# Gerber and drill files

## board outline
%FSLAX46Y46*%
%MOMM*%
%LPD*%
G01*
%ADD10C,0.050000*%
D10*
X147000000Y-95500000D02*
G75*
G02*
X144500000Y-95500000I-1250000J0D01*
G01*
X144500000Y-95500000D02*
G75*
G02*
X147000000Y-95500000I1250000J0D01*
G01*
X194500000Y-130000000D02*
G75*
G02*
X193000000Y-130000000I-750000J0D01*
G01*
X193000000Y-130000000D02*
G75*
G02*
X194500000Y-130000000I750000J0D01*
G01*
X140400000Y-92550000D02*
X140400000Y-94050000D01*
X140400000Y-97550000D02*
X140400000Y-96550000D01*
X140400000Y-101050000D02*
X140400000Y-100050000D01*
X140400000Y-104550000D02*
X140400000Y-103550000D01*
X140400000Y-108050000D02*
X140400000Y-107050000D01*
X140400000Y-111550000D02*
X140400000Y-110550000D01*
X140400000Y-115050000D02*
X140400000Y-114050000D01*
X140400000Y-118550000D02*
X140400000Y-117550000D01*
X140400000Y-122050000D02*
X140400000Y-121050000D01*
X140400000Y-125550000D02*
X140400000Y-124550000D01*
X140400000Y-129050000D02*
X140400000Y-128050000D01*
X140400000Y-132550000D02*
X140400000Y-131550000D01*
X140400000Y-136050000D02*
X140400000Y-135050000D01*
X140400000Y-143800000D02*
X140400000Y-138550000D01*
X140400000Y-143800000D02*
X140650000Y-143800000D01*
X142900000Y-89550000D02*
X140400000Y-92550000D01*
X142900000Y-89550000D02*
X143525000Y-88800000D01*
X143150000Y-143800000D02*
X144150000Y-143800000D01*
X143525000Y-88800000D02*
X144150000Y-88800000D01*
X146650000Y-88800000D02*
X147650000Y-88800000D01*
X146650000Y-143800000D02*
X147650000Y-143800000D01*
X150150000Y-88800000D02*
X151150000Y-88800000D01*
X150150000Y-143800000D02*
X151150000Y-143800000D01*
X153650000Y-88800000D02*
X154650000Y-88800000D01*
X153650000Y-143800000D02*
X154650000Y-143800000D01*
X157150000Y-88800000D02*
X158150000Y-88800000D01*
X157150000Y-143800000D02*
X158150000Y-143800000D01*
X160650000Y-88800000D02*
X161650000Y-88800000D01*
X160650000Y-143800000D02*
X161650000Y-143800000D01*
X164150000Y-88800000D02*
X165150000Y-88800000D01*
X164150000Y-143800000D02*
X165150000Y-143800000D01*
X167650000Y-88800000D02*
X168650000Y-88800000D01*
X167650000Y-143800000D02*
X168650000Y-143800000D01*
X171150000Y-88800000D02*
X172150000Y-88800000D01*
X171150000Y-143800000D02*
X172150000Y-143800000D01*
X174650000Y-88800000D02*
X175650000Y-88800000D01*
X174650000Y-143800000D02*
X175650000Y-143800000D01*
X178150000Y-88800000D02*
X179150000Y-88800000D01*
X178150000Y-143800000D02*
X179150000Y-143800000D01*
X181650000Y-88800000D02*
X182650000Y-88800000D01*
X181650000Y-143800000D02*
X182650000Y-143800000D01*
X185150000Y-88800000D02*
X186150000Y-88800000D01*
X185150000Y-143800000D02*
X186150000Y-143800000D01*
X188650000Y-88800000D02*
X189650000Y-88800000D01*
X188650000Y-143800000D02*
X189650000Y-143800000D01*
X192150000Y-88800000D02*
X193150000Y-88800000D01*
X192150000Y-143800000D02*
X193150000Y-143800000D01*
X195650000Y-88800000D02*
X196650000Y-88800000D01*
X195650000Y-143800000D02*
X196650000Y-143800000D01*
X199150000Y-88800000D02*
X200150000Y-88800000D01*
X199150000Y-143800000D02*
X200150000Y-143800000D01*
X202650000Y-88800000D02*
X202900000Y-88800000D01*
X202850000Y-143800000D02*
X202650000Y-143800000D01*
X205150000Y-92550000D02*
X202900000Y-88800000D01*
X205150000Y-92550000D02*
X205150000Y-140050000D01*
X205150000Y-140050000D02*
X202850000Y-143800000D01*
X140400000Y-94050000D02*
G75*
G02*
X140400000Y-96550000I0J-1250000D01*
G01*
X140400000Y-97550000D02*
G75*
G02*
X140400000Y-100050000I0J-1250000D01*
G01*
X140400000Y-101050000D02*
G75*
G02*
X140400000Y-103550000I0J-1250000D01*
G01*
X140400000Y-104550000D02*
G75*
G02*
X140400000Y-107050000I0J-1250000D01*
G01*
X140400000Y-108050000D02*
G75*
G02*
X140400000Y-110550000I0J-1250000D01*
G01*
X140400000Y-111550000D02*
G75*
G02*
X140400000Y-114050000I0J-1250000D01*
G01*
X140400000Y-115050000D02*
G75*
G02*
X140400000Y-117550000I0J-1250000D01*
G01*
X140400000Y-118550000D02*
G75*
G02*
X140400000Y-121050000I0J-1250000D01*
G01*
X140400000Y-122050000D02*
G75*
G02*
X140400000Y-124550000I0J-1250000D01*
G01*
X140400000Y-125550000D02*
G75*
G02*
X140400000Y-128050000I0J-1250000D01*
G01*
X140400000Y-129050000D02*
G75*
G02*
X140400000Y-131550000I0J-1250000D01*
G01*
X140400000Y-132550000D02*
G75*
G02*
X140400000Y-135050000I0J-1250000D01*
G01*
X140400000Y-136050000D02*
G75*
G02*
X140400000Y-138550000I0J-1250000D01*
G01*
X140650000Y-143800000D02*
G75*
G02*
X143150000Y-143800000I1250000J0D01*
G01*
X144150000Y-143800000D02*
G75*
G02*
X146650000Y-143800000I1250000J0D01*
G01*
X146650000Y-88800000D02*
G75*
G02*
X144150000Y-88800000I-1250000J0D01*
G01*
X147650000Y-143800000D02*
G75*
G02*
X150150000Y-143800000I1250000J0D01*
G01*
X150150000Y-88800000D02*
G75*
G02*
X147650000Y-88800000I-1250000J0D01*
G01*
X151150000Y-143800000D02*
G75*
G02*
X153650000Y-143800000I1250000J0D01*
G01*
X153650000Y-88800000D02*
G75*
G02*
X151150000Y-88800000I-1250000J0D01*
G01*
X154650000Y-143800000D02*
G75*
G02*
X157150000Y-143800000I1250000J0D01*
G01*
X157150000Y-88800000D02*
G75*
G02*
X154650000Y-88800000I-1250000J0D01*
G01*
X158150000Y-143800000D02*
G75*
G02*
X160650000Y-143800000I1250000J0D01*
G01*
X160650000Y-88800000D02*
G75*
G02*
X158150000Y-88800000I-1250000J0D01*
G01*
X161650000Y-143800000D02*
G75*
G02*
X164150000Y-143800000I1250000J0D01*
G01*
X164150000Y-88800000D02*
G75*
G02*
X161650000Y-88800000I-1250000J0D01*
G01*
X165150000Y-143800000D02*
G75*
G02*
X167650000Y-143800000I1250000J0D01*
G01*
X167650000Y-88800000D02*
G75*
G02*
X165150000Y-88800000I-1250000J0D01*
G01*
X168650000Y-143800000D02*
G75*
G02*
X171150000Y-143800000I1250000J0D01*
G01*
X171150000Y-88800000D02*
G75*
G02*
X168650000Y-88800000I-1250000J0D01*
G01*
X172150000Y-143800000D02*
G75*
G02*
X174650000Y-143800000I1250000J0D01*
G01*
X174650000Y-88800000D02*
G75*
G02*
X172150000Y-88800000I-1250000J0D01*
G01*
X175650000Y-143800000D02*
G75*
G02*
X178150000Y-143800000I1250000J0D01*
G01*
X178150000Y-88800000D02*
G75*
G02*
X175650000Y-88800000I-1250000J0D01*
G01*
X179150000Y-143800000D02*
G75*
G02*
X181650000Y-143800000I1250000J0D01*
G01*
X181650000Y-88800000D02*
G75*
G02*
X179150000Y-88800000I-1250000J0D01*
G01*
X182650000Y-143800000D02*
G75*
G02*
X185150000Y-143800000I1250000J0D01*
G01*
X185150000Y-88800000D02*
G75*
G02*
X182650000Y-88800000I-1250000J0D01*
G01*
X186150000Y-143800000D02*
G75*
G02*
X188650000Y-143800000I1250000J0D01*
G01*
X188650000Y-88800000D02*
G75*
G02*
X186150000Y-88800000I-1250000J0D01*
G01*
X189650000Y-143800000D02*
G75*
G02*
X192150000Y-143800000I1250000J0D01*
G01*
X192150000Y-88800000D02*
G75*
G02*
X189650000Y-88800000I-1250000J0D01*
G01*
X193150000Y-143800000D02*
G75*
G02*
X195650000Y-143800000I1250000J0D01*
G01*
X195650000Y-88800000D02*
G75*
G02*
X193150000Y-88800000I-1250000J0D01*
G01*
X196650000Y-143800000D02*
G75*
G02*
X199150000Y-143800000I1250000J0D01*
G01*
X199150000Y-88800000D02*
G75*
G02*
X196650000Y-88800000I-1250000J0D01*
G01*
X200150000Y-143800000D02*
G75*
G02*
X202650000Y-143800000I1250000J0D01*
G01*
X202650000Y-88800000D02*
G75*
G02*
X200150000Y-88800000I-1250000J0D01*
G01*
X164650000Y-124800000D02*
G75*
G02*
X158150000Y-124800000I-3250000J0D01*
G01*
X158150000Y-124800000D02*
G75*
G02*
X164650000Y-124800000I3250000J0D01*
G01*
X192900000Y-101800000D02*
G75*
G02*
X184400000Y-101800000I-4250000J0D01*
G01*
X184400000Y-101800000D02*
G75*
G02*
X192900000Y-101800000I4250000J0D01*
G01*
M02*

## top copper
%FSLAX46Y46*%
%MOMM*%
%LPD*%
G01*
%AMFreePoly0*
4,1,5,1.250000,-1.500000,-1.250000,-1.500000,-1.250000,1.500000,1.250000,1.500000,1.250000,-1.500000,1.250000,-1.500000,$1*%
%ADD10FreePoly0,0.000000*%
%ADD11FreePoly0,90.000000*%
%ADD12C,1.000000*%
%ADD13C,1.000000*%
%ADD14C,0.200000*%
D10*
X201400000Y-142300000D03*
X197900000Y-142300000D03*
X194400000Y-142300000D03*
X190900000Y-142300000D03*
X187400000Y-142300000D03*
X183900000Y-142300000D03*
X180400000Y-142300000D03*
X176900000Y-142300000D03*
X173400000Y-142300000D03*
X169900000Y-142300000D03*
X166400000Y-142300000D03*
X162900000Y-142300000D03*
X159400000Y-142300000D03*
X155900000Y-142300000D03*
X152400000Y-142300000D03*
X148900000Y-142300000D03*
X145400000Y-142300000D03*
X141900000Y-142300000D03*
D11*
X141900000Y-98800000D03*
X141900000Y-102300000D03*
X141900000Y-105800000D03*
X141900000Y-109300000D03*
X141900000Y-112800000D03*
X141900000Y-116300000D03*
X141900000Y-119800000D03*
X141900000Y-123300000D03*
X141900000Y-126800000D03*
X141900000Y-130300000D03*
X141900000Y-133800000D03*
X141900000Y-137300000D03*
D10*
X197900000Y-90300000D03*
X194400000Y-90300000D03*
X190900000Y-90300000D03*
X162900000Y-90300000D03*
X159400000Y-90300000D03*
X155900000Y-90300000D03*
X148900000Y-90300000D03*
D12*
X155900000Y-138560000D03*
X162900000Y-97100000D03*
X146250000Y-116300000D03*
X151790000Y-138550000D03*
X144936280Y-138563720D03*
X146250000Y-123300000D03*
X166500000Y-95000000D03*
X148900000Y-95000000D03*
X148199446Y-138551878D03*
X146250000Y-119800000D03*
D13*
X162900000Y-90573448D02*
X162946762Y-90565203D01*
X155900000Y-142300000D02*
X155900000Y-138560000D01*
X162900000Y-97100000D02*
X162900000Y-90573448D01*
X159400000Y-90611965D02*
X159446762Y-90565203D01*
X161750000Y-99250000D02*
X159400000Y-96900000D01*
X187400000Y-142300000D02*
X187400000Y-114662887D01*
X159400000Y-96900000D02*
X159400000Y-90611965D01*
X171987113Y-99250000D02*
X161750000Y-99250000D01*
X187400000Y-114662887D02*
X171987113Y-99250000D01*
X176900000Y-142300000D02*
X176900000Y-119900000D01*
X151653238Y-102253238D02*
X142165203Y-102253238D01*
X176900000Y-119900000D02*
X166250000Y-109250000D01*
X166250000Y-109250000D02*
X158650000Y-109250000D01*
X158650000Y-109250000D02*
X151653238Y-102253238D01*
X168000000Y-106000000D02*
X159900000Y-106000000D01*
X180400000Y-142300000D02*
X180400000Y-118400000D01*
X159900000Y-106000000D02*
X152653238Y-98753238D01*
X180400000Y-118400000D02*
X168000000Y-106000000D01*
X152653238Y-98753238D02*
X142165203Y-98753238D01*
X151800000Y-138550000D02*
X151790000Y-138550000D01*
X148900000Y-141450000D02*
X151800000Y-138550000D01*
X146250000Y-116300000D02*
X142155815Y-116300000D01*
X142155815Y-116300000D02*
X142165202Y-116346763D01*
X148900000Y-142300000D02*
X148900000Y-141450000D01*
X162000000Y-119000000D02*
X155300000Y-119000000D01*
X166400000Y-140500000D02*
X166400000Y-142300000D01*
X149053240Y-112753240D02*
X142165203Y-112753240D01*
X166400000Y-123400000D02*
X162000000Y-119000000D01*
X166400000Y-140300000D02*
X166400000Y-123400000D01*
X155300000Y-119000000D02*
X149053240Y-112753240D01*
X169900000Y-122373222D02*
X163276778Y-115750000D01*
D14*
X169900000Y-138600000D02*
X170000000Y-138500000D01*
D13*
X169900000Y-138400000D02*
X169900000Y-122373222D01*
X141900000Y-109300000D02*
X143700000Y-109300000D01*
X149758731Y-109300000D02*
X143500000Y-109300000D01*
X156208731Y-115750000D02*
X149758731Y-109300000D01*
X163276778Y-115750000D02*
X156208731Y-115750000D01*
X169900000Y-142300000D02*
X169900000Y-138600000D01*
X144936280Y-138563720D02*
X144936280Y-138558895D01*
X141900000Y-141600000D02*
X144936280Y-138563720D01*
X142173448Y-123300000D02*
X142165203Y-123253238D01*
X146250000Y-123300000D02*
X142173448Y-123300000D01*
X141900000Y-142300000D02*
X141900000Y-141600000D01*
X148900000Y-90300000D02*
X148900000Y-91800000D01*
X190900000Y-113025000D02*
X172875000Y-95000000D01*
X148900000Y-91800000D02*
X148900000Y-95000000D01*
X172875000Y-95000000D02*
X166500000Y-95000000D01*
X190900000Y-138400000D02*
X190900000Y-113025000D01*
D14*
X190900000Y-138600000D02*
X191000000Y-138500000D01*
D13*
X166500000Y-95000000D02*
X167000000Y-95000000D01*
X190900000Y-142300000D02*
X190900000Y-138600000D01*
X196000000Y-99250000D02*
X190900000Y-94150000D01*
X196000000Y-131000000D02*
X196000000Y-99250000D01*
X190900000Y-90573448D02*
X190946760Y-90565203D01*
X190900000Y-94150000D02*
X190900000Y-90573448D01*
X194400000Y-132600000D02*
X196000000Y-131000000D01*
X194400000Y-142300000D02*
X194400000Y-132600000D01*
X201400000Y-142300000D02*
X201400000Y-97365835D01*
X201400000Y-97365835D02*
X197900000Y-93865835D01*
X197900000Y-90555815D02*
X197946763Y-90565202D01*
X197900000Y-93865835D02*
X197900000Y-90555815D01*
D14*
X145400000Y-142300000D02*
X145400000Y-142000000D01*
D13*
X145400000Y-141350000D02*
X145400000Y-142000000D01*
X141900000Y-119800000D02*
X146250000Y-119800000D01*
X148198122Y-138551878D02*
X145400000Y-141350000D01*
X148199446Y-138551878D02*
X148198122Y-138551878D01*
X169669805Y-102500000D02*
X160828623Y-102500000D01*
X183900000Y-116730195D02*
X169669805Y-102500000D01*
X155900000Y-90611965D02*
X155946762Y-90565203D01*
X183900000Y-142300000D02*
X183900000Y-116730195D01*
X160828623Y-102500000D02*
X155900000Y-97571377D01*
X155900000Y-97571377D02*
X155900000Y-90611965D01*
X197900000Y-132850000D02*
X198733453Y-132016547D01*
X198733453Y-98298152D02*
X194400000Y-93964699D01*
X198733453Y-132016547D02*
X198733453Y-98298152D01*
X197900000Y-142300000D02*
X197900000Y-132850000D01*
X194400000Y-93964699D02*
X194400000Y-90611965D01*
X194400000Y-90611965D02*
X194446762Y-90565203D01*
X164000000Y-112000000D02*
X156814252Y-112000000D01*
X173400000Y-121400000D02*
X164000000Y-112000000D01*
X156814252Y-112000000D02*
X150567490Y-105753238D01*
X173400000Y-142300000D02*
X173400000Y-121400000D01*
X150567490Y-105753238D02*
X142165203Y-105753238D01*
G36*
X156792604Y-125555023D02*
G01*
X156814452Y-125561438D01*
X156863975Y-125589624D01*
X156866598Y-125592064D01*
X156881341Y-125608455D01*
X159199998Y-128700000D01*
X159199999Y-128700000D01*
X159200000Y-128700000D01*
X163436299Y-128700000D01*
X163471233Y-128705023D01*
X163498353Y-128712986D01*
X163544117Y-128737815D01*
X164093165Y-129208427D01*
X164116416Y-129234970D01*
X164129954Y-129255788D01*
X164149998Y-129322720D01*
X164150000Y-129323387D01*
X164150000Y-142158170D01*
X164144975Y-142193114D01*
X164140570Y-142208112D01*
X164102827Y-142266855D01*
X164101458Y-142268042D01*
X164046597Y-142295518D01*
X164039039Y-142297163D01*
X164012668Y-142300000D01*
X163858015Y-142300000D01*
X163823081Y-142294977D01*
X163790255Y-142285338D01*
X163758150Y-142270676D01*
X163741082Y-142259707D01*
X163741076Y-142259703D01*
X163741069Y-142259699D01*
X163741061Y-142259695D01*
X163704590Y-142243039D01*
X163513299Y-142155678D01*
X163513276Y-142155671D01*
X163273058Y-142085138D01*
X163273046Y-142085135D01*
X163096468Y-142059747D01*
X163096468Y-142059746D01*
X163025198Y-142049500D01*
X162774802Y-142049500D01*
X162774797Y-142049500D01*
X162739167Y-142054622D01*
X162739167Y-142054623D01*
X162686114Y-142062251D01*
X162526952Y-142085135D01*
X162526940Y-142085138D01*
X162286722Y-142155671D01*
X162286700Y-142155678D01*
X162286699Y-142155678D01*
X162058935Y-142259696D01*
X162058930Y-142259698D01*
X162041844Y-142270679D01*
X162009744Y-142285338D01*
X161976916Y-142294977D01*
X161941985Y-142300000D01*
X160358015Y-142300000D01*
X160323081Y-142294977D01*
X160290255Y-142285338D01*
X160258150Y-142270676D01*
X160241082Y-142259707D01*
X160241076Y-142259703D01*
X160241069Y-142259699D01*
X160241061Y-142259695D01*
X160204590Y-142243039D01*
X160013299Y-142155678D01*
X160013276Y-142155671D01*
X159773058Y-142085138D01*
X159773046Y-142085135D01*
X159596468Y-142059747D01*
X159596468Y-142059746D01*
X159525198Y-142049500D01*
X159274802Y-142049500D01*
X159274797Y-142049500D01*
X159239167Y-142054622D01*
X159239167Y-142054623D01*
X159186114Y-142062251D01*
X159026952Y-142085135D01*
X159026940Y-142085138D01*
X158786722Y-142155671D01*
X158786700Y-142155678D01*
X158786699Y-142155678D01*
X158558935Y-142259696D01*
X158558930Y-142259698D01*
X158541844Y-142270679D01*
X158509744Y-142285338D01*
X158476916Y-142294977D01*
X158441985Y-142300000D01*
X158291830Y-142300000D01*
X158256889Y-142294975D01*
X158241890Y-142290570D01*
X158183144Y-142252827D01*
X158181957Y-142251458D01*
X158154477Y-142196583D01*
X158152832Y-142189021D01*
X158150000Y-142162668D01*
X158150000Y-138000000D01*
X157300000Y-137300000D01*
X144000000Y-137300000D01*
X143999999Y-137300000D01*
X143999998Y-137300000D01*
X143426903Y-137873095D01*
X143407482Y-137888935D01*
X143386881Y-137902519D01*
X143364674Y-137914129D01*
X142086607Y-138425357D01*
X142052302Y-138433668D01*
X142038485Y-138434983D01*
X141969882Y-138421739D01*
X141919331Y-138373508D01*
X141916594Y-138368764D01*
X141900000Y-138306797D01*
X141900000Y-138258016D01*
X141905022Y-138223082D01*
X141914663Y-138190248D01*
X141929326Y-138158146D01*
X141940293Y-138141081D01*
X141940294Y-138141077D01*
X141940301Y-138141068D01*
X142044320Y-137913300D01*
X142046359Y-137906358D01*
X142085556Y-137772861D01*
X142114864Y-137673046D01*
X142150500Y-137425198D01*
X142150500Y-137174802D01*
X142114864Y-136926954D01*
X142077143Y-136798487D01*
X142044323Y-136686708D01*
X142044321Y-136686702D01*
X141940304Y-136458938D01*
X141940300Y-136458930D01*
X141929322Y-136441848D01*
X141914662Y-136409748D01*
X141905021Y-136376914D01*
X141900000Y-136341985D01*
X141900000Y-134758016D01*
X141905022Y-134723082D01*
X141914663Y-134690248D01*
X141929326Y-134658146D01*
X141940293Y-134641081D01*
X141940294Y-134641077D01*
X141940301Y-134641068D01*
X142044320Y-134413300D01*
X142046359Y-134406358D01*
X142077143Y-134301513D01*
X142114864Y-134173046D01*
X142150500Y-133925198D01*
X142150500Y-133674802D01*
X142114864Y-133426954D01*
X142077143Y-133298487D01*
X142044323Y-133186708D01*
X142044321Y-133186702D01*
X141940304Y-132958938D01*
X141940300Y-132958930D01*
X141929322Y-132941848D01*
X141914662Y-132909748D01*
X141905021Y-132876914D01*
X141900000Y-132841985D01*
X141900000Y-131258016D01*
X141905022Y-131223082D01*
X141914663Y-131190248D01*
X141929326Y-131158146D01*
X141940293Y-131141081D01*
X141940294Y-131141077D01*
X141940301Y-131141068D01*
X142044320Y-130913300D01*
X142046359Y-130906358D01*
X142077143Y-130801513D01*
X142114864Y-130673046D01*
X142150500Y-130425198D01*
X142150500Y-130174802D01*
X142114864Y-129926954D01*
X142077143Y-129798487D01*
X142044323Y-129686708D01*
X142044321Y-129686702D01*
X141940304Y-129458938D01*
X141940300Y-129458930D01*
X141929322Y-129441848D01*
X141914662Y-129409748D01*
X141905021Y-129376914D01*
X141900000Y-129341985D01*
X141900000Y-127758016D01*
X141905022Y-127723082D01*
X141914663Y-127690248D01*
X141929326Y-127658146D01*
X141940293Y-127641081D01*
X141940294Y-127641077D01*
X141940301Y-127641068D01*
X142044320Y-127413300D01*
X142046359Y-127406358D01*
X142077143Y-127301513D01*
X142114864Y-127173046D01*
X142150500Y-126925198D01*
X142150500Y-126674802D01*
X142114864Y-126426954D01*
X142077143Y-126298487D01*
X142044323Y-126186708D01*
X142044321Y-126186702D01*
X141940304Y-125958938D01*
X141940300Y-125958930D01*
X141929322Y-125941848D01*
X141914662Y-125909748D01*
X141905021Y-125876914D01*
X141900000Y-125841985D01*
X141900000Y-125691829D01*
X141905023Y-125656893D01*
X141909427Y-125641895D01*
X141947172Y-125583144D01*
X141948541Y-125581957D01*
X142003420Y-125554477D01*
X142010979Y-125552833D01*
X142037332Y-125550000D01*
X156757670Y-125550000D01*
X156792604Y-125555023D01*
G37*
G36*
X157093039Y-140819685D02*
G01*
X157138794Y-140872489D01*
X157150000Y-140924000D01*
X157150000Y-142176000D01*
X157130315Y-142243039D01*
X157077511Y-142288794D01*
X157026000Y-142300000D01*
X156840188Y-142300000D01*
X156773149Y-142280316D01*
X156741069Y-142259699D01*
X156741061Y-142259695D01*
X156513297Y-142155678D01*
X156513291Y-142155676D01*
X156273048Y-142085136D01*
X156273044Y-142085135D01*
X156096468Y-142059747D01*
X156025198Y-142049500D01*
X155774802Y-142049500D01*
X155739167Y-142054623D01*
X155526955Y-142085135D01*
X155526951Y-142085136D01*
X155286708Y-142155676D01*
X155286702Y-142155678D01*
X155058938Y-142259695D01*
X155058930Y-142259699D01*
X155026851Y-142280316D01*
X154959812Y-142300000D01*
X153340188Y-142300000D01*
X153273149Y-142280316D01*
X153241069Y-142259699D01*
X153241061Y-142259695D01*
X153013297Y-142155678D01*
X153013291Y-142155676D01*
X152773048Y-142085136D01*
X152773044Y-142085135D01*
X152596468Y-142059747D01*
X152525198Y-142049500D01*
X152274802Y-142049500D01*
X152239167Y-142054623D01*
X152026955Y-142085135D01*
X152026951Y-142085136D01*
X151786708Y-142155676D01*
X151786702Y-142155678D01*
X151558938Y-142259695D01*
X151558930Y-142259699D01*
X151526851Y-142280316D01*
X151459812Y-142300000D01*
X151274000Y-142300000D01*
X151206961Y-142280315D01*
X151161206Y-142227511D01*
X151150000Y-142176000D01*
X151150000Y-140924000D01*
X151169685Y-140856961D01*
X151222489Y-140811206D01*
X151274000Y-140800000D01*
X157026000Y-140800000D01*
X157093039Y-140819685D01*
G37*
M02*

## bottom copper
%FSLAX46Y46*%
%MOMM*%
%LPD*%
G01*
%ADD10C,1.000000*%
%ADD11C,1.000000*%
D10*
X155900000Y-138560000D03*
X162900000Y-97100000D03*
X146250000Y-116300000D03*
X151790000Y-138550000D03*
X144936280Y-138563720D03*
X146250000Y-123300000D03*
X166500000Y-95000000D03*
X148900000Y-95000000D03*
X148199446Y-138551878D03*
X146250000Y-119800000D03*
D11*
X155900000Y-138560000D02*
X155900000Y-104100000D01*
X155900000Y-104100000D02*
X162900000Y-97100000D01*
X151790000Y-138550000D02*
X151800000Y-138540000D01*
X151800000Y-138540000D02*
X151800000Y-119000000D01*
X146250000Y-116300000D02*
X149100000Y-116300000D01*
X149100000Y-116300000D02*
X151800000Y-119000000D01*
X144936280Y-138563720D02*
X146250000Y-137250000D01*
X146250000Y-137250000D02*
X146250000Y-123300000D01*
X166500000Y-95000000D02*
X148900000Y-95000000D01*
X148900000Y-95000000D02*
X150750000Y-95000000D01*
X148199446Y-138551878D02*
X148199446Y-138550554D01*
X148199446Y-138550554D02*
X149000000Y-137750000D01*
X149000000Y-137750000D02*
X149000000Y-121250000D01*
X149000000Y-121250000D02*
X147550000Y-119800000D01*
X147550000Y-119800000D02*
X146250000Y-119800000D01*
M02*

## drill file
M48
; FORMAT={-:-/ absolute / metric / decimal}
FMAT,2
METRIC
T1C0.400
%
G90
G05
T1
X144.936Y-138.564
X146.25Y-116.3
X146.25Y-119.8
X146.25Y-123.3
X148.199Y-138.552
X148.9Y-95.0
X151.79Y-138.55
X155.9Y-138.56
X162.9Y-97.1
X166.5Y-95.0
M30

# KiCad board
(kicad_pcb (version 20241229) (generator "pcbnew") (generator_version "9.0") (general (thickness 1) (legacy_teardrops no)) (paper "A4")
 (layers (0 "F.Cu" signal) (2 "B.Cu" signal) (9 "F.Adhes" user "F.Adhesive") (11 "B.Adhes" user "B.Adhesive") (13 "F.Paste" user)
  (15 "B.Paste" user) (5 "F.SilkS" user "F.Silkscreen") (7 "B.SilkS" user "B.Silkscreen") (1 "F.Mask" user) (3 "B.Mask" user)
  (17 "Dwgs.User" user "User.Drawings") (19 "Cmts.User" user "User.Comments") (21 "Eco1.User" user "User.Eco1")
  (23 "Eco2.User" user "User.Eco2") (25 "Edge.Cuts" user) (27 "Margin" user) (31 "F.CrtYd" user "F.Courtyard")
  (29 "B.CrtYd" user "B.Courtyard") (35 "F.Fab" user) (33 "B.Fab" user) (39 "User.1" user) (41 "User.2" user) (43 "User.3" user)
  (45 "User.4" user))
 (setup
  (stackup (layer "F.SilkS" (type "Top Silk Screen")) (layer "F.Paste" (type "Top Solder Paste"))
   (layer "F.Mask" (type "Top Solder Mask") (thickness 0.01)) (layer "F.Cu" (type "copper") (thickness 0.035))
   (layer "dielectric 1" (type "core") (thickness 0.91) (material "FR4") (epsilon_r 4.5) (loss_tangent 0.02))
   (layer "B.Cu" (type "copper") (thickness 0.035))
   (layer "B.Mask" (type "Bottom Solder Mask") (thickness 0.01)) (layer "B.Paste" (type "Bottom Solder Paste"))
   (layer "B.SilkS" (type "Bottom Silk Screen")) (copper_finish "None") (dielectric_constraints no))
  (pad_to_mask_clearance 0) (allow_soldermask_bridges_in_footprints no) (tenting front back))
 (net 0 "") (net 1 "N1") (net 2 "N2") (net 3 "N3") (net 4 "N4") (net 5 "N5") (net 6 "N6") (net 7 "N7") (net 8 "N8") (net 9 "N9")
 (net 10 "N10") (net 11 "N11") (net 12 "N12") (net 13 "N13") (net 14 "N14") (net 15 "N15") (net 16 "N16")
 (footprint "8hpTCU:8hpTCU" (layer "F.Cu") (at 176.4 105.8)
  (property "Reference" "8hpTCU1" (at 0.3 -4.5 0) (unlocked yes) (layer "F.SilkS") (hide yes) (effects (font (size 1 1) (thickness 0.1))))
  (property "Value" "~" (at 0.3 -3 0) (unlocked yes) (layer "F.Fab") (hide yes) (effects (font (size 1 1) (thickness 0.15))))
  (fp_line (start -36 -13.25) (end -36 -11.75) (stroke (width 0.05) (type default)) (layer "Edge.Cuts"))
  (fp_line (start -36 -8.25) (end -36 -9.25) (stroke (width 0.05) (type default)) (layer "Edge.Cuts"))
  (fp_line (start -36 -4.75) (end -36 -5.75) (stroke (width 0.05) (type default)) (layer "Edge.Cuts"))
  (fp_line (start -36 -1.25) (end -36 -2.25) (stroke (width 0.05) (type default)) (layer "Edge.Cuts"))
  (fp_line (start -36 2.25) (end -36 1.25) (stroke (width 0.05) (type default)) (layer "Edge.Cuts"))
  (fp_line (start -36 5.75) (end -36 4.75) (stroke (width 0.05) (type default)) (layer "Edge.Cuts"))
  (fp_line (start -36 9.25) (end -36 8.25) (stroke (width 0.05) (type default)) (layer "Edge.Cuts"))
  (fp_line (start -36 12.75) (end -36 11.75) (stroke (width 0.05) (type default)) (layer "Edge.Cuts"))
  (fp_line (start -36 16.25) (end -36 15.25) (stroke (width 0.05) (type default)) (layer "Edge.Cuts"))
  (fp_line (start -36 19.75) (end -36 18.75) (stroke (width 0.05) (type default)) (layer "Edge.Cuts"))
  (fp_line (start -36 23.25) (end -36 22.25) (stroke (width 0.05) (type default)) (layer "Edge.Cuts"))
  (fp_line (start -36 26.75) (end -36 25.75) (stroke (width 0.05) (type default)) (layer "Edge.Cuts"))
  (fp_line (start -36 30.25) (end -36 29.25) (stroke (width 0.05) (type default)) (layer "Edge.Cuts"))
  (fp_line (start -36 38) (end -36 32.75) (stroke (width 0.05) (type default)) (layer "Edge.Cuts"))
  (fp_line (start -36 38) (end -35.75 38) (stroke (width 0.05) (type default)) (layer "Edge.Cuts"))
  (fp_line (start -33.5 -16.25) (end -36 -13.25) (stroke (width 0.05) (type default)) (layer "Edge.Cuts"))
  (fp_line (start -33.5 -16.25) (end -32.875 -17) (stroke (width 0.05) (type default)) (layer "Edge.Cuts"))
  (fp_line (start -33.25 38) (end -32.25 38) (stroke (width 0.05) (type default)) (layer "Edge.Cuts"))
  (fp_line (start -32.875 -17) (end -32.25 -17) (stroke (width 0.05) (type default)) (layer "Edge.Cuts"))
  (fp_line (start -29.75 -17) (end -28.75 -17) (stroke (width 0.05) (type default)) (layer "Edge.Cuts"))
  (fp_line (start -29.75 38) (end -28.75 38) (stroke (width 0.05) (type default)) (layer "Edge.Cuts"))
  (fp_line (start -26.25 -17) (end -25.25 -17) (stroke (width 0.05) (type default)) (layer "Edge.Cuts"))
  (fp_line (start -26.25 38) (end -25.25 38) (stroke (width 0.05) (type default)) (layer "Edge.Cuts"))
  (fp_line (start -22.75 -17) (end -21.75 -17) (stroke (width 0.05) (type default)) (layer "Edge.Cuts"))
  (fp_line (start -22.75 38) (end -21.75 38) (stroke (width 0.05) (type default)) (layer "Edge.Cuts"))
  (fp_line (start -19.25 -17) (end -18.25 -17) (stroke (width 0.05) (type default)) (layer "Edge.Cuts"))
  (fp_line (start -19.25 38) (end -18.25 38) (stroke (width 0.05) (type default)) (layer "Edge.Cuts"))
  (fp_line (start -15.75 -17) (end -14.75 -17) (stroke (width 0.05) (type default)) (layer "Edge.Cuts"))
  (fp_line (start -15.75 38) (end -14.75 38) (stroke (width 0.05) (type default)) (layer "Edge.Cuts"))
  (fp_line (start -12.25 -17) (end -11.25 -17) (stroke (width 0.05) (type default)) (layer "Edge.Cuts"))
  (fp_line (start -12.25 38) (end -11.25 38) (stroke (width 0.05) (type default)) (layer "Edge.Cuts"))
  (fp_line (start -8.75 -17) (end -7.75 -17) (stroke (width 0.05) (type default)) (layer "Edge.Cuts"))
  (fp_line (start -8.75 38) (end -7.75 38) (stroke (width 0.05) (type default)) (layer "Edge.Cuts"))
  (fp_line (start -5.25 -17) (end -4.25 -17) (stroke (width 0.05) (type default)) (layer "Edge.Cuts"))
  (fp_line (start -5.25 38) (end -4.25 38) (stroke (width 0.05) (type default)) (layer "Edge.Cuts"))
  (fp_line (start -1.75 -17) (end -0.75 -17) (stroke (width 0.05) (type default)) (layer "Edge.Cuts"))
  (fp_line (start -1.75 38) (end -0.75 38) (stroke (width 0.05) (type default)) (layer "Edge.Cuts"))
  (fp_line (start 1.75 -17) (end 2.75 -17) (stroke (width 0.05) (type default)) (layer "Edge.Cuts"))
  (fp_line (start 1.75 38) (end 2.75 38) (stroke (width 0.05) (type default)) (layer "Edge.Cuts"))
  (fp_line (start 5.25 -17) (end 6.25 -17) (stroke (width 0.05) (type default)) (layer "Edge.Cuts"))
  (fp_line (start 5.25 38) (end 6.25 38) (stroke (width 0.05) (type default)) (layer "Edge.Cuts"))
  (fp_line (start 8.75 -17) (end 9.75 -17) (stroke (width 0.05) (type default)) (layer "Edge.Cuts"))
  (fp_line (start 8.75 38) (end 9.75 38) (stroke (width 0.05) (type default)) (layer "Edge.Cuts"))
  (fp_line (start 12.25 -17) (end 13.25 -17) (stroke (width 0.05) (type default)) (layer "Edge.Cuts"))
  (fp_line (start 12.25 38) (end 13.25 38) (stroke (width 0.05) (type default)) (layer "Edge.Cuts"))
  (fp_line (start 15.75 -17) (end 16.75 -17) (stroke (width 0.05) (type default)) (layer "Edge.Cuts"))
  (fp_line (start 15.75 38) (end 16.75 38) (stroke (width 0.05) (type default)) (layer "Edge.Cuts"))
  (fp_line (start 19.25 -17) (end 20.25 -17) (stroke (width 0.05) (type default)) (layer "Edge.Cuts"))
  (fp_line (start 19.25 38) (end 20.25 38) (stroke (width 0.05) (type default)) (layer "Edge.Cuts"))
  (fp_line (start 22.75 -17) (end 23.75 -17) (stroke (width 0.05) (type default)) (layer "Edge.Cuts"))
  (fp_line (start 22.75 38) (end 23.75 38) (stroke (width 0.05) (type default)) (layer "Edge.Cuts"))
  (fp_line (start 26.25 -17) (end 26.5 -17) (stroke (width 0.05) (type default)) (layer "Edge.Cuts"))
  (fp_line (start 26.45 38) (end 26.25 38) (stroke (width 0.05) (type default)) (layer "Edge.Cuts"))
  (fp_line (start 28.75 -13.25) (end 26.5 -17) (stroke (width 0.05) (type default)) (layer "Edge.Cuts"))
  (fp_line (start 28.75 -13.25) (end 28.75 34.25) (stroke (width 0.05) (type default)) (layer "Edge.Cuts"))
  (fp_line (start 28.75 34.25) (end 26.45 38) (stroke (width 0.05) (type default)) (layer "Edge.Cuts"))
  (fp_arc (start -36 -11.75) (mid -34.75 -10.5) (end -36 -9.25) (stroke (width 0.05) (type default)) (layer "Edge.Cuts"))
  (fp_arc (start -36 -8.25) (mid -34.75 -7) (end -36 -5.75) (stroke (width 0.05) (type default)) (layer "Edge.Cuts"))
  (fp_arc (start -36 -4.75) (mid -34.75 -3.5) (end -36 -2.25) (stroke (width 0.05) (type default)) (layer "Edge.Cuts"))
  (fp_arc (start -36 -1.25) (mid -34.75 0) (end -36 1.25) (stroke (width 0.05) (type default)) (layer "Edge.Cuts"))
  (fp_arc (start -36 2.25) (mid -34.75 3.5) (end -36 4.75) (stroke (width 0.05) (type default)) (layer "Edge.Cuts"))
  (fp_arc (start -36 5.75) (mid -34.75 7) (end -36 8.25) (stroke (width 0.05) (type default)) (layer "Edge.Cuts"))
  (fp_arc (start -36 9.25) (mid -34.75 10.5) (end -36 11.75) (stroke (width 0.05) (type default)) (layer "Edge.Cuts"))
  (fp_arc (start -36 12.75) (mid -34.75 14) (end -36 15.25) (stroke (width 0.05) (type default)) (layer "Edge.Cuts"))
  (fp_arc (start -36 16.25) (mid -34.75 17.5) (end -36 18.75) (stroke (width 0.05) (type default)) (layer "Edge.Cuts"))
  (fp_arc (start -36 19.75) (mid -34.75 21) (end -36 22.25) (stroke (width 0.05) (type default)) (layer "Edge.Cuts"))
  (fp_arc (start -36 23.25) (mid -34.75 24.5) (end -36 25.75) (stroke (width 0.05) (type default)) (layer "Edge.Cuts"))
  (fp_arc (start -36 26.75) (mid -34.75 28) (end -36 29.25) (stroke (width 0.05) (type default)) (layer "Edge.Cuts"))
  (fp_arc (start -36 30.25) (mid -34.75 31.5) (end -36 32.75) (stroke (width 0.05) (type default)) (layer "Edge.Cuts"))
  (fp_arc (start -35.75 38) (mid -34.5 36.75) (end -33.25 38) (stroke (width 0.05) (type default)) (layer "Edge.Cuts"))
  (fp_arc (start -32.25 38) (mid -31 36.75) (end -29.75 38) (stroke (width 0.05) (type default)) (layer "Edge.Cuts"))
  (fp_arc (start -29.75 -17) (mid -31 -15.75) (end -32.25 -17) (stroke (width 0.05) (type default)) (layer "Edge.Cuts"))
  (fp_arc (start -28.75 38) (mid -27.5 36.75) (end -26.25 38) (stroke (width 0.05) (type default)) (layer "Edge.Cuts"))
  (fp_arc (start -26.25 -17) (mid -27.5 -15.75) (end -28.75 -17) (stroke (width 0.05) (type default)) (layer "Edge.Cuts"))
  (fp_arc (start -25.25 38) (mid -24 36.75) (end -22.75 38) (stroke (width 0.05) (type default)) (layer "Edge.Cuts"))
  (fp_arc (start -22.75 -17) (mid -24 -15.75) (end -25.25 -17) (stroke (width 0.05) (type default)) (layer "Edge.Cuts"))
  (fp_arc (start -21.75 38) (mid -20.5 36.75) (end -19.25 38) (stroke (width 0.05) (type default)) (layer "Edge.Cuts"))
  (fp_arc (start -19.25 -17) (mid -20.5 -15.75) (end -21.75 -17) (stroke (width 0.05) (type default)) (layer "Edge.Cuts"))
  (fp_arc (start -18.25 38) (mid -17 36.75) (end -15.75 38) (stroke (width 0.05) (type default)) (layer "Edge.Cuts"))
  (fp_arc (start -15.75 -17) (mid -17 -15.75) (end -18.25 -17) (stroke (width 0.05) (type default)) (layer "Edge.Cuts"))
  (fp_arc (start -14.75 38) (mid -13.5 36.75) (end -12.25 38) (stroke (width 0.05) (type default)) (layer "Edge.Cuts"))
  (fp_arc (start -12.25 -17) (mid -13.5 -15.75) (end -14.75 -17) (stroke (width 0.05) (type default)) (layer "Edge.Cuts"))
  (fp_arc (start -11.25 38) (mid -10 36.75) (end -8.75 38) (stroke (width 0.05) (type default)) (layer "Edge.Cuts"))
  (fp_arc (start -8.75 -17) (mid -10 -15.75) (end -11.25 -17) (stroke (width 0.05) (type default)) (layer "Edge.Cuts"))
  (fp_arc (start -7.75 38) (mid -6.5 36.75) (end -5.25 38) (stroke (width 0.05) (type default)) (layer "Edge.Cuts"))
  (fp_arc (start -5.25 -17) (mid -6.5 -15.75) (end -7.75 -17) (stroke (width 0.05) (type default)) (layer "Edge.Cuts"))
  (fp_arc (start -4.25 38) (mid -3 36.75) (end -1.75 38) (stroke (width 0.05) (type default)) (layer "Edge.Cuts"))
  (fp_arc (start -1.75 -17) (mid -3 -15.75) (end -4.25 -17) (stroke (width 0.05) (type default)) (layer "Edge.Cuts"))
  (fp_arc (start -0.75 38) (mid 0.5 36.75) (end 1.75 38) (stroke (width 0.05) (type default)) (layer "Edge.Cuts"))
  (fp_arc (start 1.75 -17) (mid 0.5 -15.75) (end -0.75 -17) (stroke (width 0.05) (type default)) (layer "Edge.Cuts"))
  (fp_arc (start 2.75 38) (mid 4 36.75) (end 5.25 38) (stroke (width 0.05) (type default)) (layer "Edge.Cuts"))
  (fp_arc (start 5.25 -17) (mid 4 -15.75) (end 2.75 -17) (stroke (width 0.05) (type default)) (layer "Edge.Cuts"))
  (fp_arc (start 6.25 38) (mid 7.5 36.75) (end 8.75 38) (stroke (width 0.05) (type default)) (layer "Edge.Cuts"))
  (fp_arc (start 8.75 -17) (mid 7.5 -15.75) (end 6.25 -17) (stroke (width 0.05) (type default)) (layer "Edge.Cuts"))
  (fp_arc (start 9.75 38) (mid 11 36.75) (end 12.25 38) (stroke (width 0.05) (type default)) (layer "Edge.Cuts"))
  (fp_arc (start 12.25 -17) (mid 11 -15.75) (end 9.75 -17) (stroke (width 0.05) (type default)) (layer "Edge.Cuts"))
  (fp_arc (start 13.25 38) (mid 14.5 36.75) (end 15.75 38) (stroke (width 0.05) (type default)) (layer "Edge.Cuts"))
  (fp_arc (start 15.75 -17) (mid 14.5 -15.75) (end 13.25 -17) (stroke (width 0.05) (type default)) (layer "Edge.Cuts"))
  (fp_arc (start 16.75 38) (mid 18 36.75) (end 19.25 38) (stroke (width 0.05) (type default)) (layer "Edge.Cuts"))
  (fp_arc (start 19.25 -17) (mid 18 -15.75) (end 16.75 -17) (stroke (width 0.05) (type default)) (layer "Edge.Cuts"))
  (fp_arc (start 20.25 38) (mid 21.5 36.75) (end 22.75 38) (stroke (width 0.05) (type default)) (layer "Edge.Cuts"))
  (fp_arc (start 22.75 -17) (mid 21.5 -15.75) (end 20.25 -17) (stroke (width 0.05) (type default)) (layer "Edge.Cuts"))
  (fp_arc (start 23.75 38) (mid 25 36.75) (end 26.25 38) (stroke (width 0.05) (type default)) (layer "Edge.Cuts"))
  (fp_arc (start 26.25 -17) (mid 25 -15.75) (end 23.75 -17) (stroke (width 0.05) (type default)) (layer "Edge.Cuts"))
  (fp_circle (center -15 19) (end -11.75 19) (stroke (width 0.05) (type default)) (fill no) (layer "Edge.Cuts"))
  (fp_circle (center 12.25 -4) (end 12.25 -8.25) (stroke (width 0.05) (type default)) (fill no) (layer "Edge.Cuts"))
  (pad "A1" smd custom (at 25 36.5) (size 2.5 3) (layers "F.Cu" "F.Mask" "F.Paste") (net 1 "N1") (options (clearance outline) (anchor rect))
   (primitives))
  (pad "A2" smd custom (at 21.5 36.5) (size 2.5 3) (layers "F.Cu" "F.Mask" "F.Paste") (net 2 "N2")
   (options (clearance outline) (anchor rect)) (primitives))
  (pad "A3" smd custom (at 18 36.5) (size 2.5 3) (layers "F.Cu" "F.Mask" "F.Paste") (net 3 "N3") (options (clearance outline) (anchor rect))
   (primitives))
  (pad "A4" smd custom (at 14.5 36.5) (size 2.5 3) (layers "F.Cu" "F.Mask" "F.Paste") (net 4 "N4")
   (options (clearance outline) (anchor rect)) (primitives))
  (pad "A5" smd custom (at 11 36.5) (size 2.5 3) (layers "F.Cu" "F.Mask" "F.Paste") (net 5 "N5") (options (clearance outline) (anchor rect))
   (primitives))
  (pad "A6" smd custom (at 7.5 36.5) (size 2.5 3) (layers "F.Cu" "F.Mask" "F.Paste") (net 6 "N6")
   (options (clearance outline) (anchor rect)) (primitives))
  (pad "A7" smd custom (at 4 36.5) (size 2.5 3) (layers "F.Cu" "F.Mask" "F.Paste") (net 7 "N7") (options (clearance outline) (anchor rect))
   (primitives))
  (pad "A8" smd custom (at 0.5 36.5) (size 2.5 3) (layers "F.Cu" "F.Mask" "F.Paste") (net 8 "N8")
   (options (clearance outline) (anchor rect)) (primitives))
  (pad "A9" smd custom (at -3 36.5) (size 2.5 3) (layers "F.Cu" "F.Mask" "F.Paste") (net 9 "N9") (options (clearance outline) (anchor rect))
   (primitives))
  (pad "A10" smd custom (at -6.5 36.5) (size 2.5 3) (layers "F.Cu" "F.Mask" "F.Paste") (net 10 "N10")
   (options (clearance outline) (anchor rect)) (primitives))
  (pad "A11" smd custom (at -10 36.5) (size 2.5 3) (layers "F.Cu" "F.Mask" "F.Paste") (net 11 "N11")
   (options (clearance outline) (anchor rect)) (primitives))
  (pad "A12" smd custom (at -13.5 36.5) (size 2.5 3) (layers "F.Cu" "F.Mask" "F.Paste") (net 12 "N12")
   (options (clearance outline) (anchor rect)) (primitives))
  (pad "A13" smd custom (at -17 36.5) (size 2.5 3) (layers "F.Cu" "F.Mask" "F.Paste") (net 12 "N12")
   (options (clearance outline) (anchor rect)) (primitives))
  (pad "A14" smd custom (at -20.5 36.5) (size 2.5 3) (layers "F.Cu" "F.Mask" "F.Paste") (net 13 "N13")
   (options (clearance outline) (anchor rect)) (primitives))
  (pad "A15" smd custom (at -24 36.5) (size 2.5 3) (layers "F.Cu" "F.Mask" "F.Paste") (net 13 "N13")
   (options (clearance outline) (anchor rect)) (primitives))
  (pad "A16" smd custom (at -27.5 36.5) (size 2.5 3) (layers "F.Cu" "F.Mask" "F.Paste") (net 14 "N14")
   (options (clearance outline) (anchor rect)) (primitives))
  (pad "A17" smd custom (at -31 36.5) (size 2.5 3) (layers "F.Cu" "F.Mask" "F.Paste") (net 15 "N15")
   (options (clearance outline) (anchor rect)) (primitives))
  (pad "A18" smd custom (at -34.5 36.5) (size 2.5 3) (layers "F.Cu" "F.Mask" "F.Paste") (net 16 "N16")
   (options (clearance outline) (anchor rect)) (primitives))
  (pad "B2" smd custom (at -34.5 -7 90) (size 2.5 3) (layers "F.Cu" "F.Mask" "F.Paste") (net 7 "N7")
   (options (clearance outline) (anchor rect)) (primitives))
  (pad "B3" smd custom (at -34.5 -3.5 90) (size 2.5 3) (layers "F.Cu" "F.Mask" "F.Paste") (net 8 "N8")
   (options (clearance outline) (anchor rect)) (primitives))
  (pad "B4" smd custom (at -34.5 0 90) (size 2.5 3) (layers "F.Cu" "F.Mask" "F.Paste") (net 9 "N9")
   (options (clearance outline) (anchor rect)) (primitives))
  (pad "B5" smd custom (at -34.5 3.5 90) (size 2.5 3) (layers "F.Cu" "F.Mask" "F.Paste") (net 10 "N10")
   (options (clearance outline) (anchor rect)) (primitives))
  (pad "B6" smd custom (at -34.5 7 90) (size 2.5 3) (layers "F.Cu" "F.Mask" "F.Paste") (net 11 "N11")
   (options (clearance outline) (anchor rect)) (primitives))
  (pad "B7" smd custom (at -34.5 10.5 90) (size 2.5 3) (layers "F.Cu" "F.Mask" "F.Paste") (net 14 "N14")
   (options (clearance outline) (anchor rect)) (primitives))
  (pad "B8" smd custom (at -34.5 14 90) (size 2.5 3) (layers "F.Cu" "F.Mask" "F.Paste") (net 15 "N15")
   (options (clearance outline) (anchor rect)) (primitives))
  (pad "B9" smd custom (at -34.5 17.5 90) (size 2.5 3) (layers "F.Cu" "F.Mask" "F.Paste") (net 16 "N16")
   (options (clearance outline) (anchor rect)) (primitives))
  (pad "B10" smd custom (at -34.5 21 90) (size 2.5 3) (layers "F.Cu" "F.Mask" "F.Paste") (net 12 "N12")
   (options (clearance outline) (anchor rect)) (primitives))
  (pad "B11" smd custom (at -34.5 24.5 90) (size 2.5 3) (layers "F.Cu" "F.Mask" "F.Paste") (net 12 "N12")
   (options (clearance outline) (anchor rect)) (primitives))
  (pad "B12" smd custom (at -34.5 28 90) (size 2.5 3) (layers "F.Cu" "F.Mask" "F.Paste") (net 12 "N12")
   (options (clearance outline) (anchor rect)) (primitives))
  (pad "B13" smd custom (at -34.5 31.5 90) (size 2.5 3) (layers "F.Cu" "F.Mask" "F.Paste") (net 12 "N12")
   (options (clearance outline) (anchor rect)) (primitives))
  (pad "C2" smd custom (at 21.5 -15.5) (size 2.5 3) (layers "F.Cu" "F.Mask" "F.Paste") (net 1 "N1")
   (options (clearance outline) (anchor rect)) (primitives))
  (pad "C3" smd custom (at 18 -15.5) (size 2.5 3) (layers "F.Cu" "F.Mask" "F.Paste") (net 2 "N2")
   (options (clearance outline) (anchor rect)) (primitives))
  (pad "C4" smd custom (at 14.5 -15.5) (size 2.5 3) (layers "F.Cu" "F.Mask" "F.Paste") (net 3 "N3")
   (options (clearance outline) (anchor rect)) (primitives))
  (pad "C12" smd custom (at -13.5 -15.5) (size 2.5 3) (layers "F.Cu" "F.Mask" "F.Paste") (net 13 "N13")
   (options (clearance outline) (anchor rect)) (primitives))
  (pad "C13" smd custom (at -17 -15.5) (size 2.5 3) (layers "F.Cu" "F.Mask" "F.Paste") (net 5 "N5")
   (options (clearance outline) (anchor rect)) (primitives))
  (pad "C14" smd custom (at -20.5 -15.5) (size 2.5 3) (layers "F.Cu" "F.Mask" "F.Paste") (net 6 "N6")
   (options (clearance outline) (anchor rect)) (primitives))
  (pad "C16" smd custom (at -27.5 -15.5) (size 2.5 3) (layers "F.Cu" "F.Mask" "F.Paste") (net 4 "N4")
   (options (clearance outline) (anchor rect)) (primitives)))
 (gr_circle (center 145.75 95.5) (end 147 95.5) (stroke (width 0.05) (type default)) (fill no) (layer "Edge.Cuts"))
 (gr_circle (center 193.75 130) (end 194.5 130) (stroke (width 0.05) (type default)) (fill no) (layer "Edge.Cuts"))
 (segment (start 162.9 90.573448) (end 162.946762 90.565203) (width 1) (layer "F.Cu") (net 13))
 (segment (start 155.9 142.3) (end 155.9 138.56) (width 1) (layer "F.Cu") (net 13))
 (segment (start 162.9 97.1) (end 162.9 90.573448) (width 1) (layer "F.Cu") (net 13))
 (via blind (at 155.9 138.56) (size 1) (drill 0.4) (layers "F.Cu" "B.Cu") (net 13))
 (via blind (at 162.9 97.1) (size 1) (drill 0.4) (layers "F.Cu" "B.Cu") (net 13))
 (segment (start 155.9 138.56) (end 155.9 104.1) (width 1) (layer "B.Cu") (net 13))
 (segment (start 155.9 104.1) (end 162.9 97.1) (width 1) (layer "B.Cu") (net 13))
 (segment (start 159.4 90.611965) (end 159.446762 90.565203) (width 1) (layer "F.Cu") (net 5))
 (segment (start 161.75 99.25) (end 159.4 96.9) (width 1) (layer "F.Cu") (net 5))
 (segment (start 187.4 142.3) (end 187.4 114.662887) (width 1) (layer "F.Cu") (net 5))
 (segment (start 159.4 96.9) (end 159.4 90.611965) (width 1) (layer "F.Cu") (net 5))
 (segment (start 171.987113 99.25) (end 161.75 99.25) (width 1) (layer "F.Cu") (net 5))
 (segment (start 187.4 114.662887) (end 171.987113 99.25) (width 1) (layer "F.Cu") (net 5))
 (segment (start 176.9 142.3) (end 176.9 119.9) (width 1) (layer "F.Cu") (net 8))
 (segment (start 151.653238 102.253238) (end 142.165203 102.253238) (width 1) (layer "F.Cu") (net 8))
 (segment (start 176.9 119.9) (end 166.25 109.25) (width 1) (layer "F.Cu") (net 8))
 (segment (start 166.25 109.25) (end 158.65 109.25) (width 1) (layer "F.Cu") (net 8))
 (segment (start 158.65 109.25) (end 151.653238 102.253238) (width 1) (layer "F.Cu") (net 8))
 (segment (start 168 106) (end 159.9 106) (width 1) (layer "F.Cu") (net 7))
 (segment (start 180.4 142.3) (end 180.4 118.4) (width 1) (layer "F.Cu") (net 7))
 (segment (start 159.9 106) (end 152.653238 98.753238) (width 1) (layer "F.Cu") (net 7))
 (segment (start 180.4 118.4) (end 168 106) (width 1) (layer "F.Cu") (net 7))
 (segment (start 152.653238 98.753238) (end 142.165203 98.753238) (width 1) (layer "F.Cu") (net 7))
 (segment (start 151.8 138.55) (end 151.79 138.55) (width 1) (layer "F.Cu") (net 14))
 (segment (start 148.9 141.45) (end 151.8 138.55) (width 1) (layer "F.Cu") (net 14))
 (segment (start 146.25 116.3) (end 142.155815 116.3) (width 1) (layer "F.Cu") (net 14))
 (segment (start 142.155815 116.3) (end 142.165202 116.346763) (width 1) (layer "F.Cu") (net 14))
 (segment (start 148.9 142.3) (end 148.9 141.45) (width 1) (layer "F.Cu") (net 14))
 (via blind (at 146.25 116.3) (size 1) (drill 0.4) (layers "F.Cu" "B.Cu") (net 14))
 (via blind (at 151.79 138.55) (size 1) (drill 0.4) (layers "F.Cu" "B.Cu") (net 14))
 (segment (start 151.79 138.55) (end 151.8 138.54) (width 1) (layer "B.Cu") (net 14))
 (segment (start 151.8 138.54) (end 151.8 119) (width 1) (layer "B.Cu") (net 14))
 (segment (start 146.25 116.3) (end 149.1 116.3) (width 1) (layer "B.Cu") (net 14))
 (segment (start 149.1 116.3) (end 151.8 119) (width 1) (layer "B.Cu") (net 14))
 (segment (start 162 119) (end 155.3 119) (width 1) (layer "F.Cu") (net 11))
 (segment (start 166.4 140.5) (end 166.4 142.3) (width 1) (layer "F.Cu") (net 11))
 (segment (start 149.05324 112.75324) (end 142.165203 112.75324) (width 1) (layer "F.Cu") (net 11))
 (segment (start 166.4 123.4) (end 162 119) (width 1) (layer "F.Cu") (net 11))
 (segment (start 166.4 140.3) (end 166.4 123.4) (width 1) (layer "F.Cu") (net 11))
 (segment (start 155.3 119) (end 149.05324 112.75324) (width 1) (layer "F.Cu") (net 11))
 (segment (start 169.9 122.373222) (end 163.276778 115.75) (width 1) (layer "F.Cu") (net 10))
 (segment (start 169.9 138.6) (end 170 138.5) (width 0.2) (layer "F.Cu") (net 10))
 (segment (start 169.9 138.4) (end 169.9 122.373222) (width 1) (layer "F.Cu") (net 10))
 (segment (start 141.9 109.3) (end 143.7 109.3) (width 1) (layer "F.Cu") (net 10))
 (segment (start 149.758731 109.3) (end 143.5 109.3) (width 1) (layer "F.Cu") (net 10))
 (segment (start 156.208731 115.75) (end 149.758731 109.3) (width 1) (layer "F.Cu") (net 10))
 (segment (start 163.276778 115.75) (end 156.208731 115.75) (width 1) (layer "F.Cu") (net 10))
 (segment (start 169.9 142.3) (end 169.9 138.6) (width 1) (layer "F.Cu") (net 10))
 (segment (start 144.93628 138.56372) (end 144.93628 138.558895) (width 1) (layer "F.Cu") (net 16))
 (segment (start 141.9 141.6) (end 144.93628 138.56372) (width 1) (layer "F.Cu") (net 16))
 (segment (start 142.173448 123.3) (end 142.165203 123.253238) (width 1) (layer "F.Cu") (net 16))
 (segment (start 146.25 123.3) (end 142.173448 123.3) (width 1) (layer "F.Cu") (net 16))
 (segment (start 141.9 142.3) (end 141.9 141.6) (width 1) (layer "F.Cu") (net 16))
 (via blind (at 144.93628 138.56372) (size 1) (drill 0.4) (layers "F.Cu" "B.Cu") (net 16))
 (via blind (at 146.25 123.3) (size 1) (drill 0.4) (layers "F.Cu" "B.Cu") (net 16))
 (segment (start 144.93628 138.56372) (end 146.25 137.25) (width 1) (layer "B.Cu") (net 16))
 (segment (start 146.25 137.25) (end 146.25 123.3) (width 1) (layer "B.Cu") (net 16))
 (segment (start 148.9 90.3) (end 148.9 91.8) (width 1) (layer "F.Cu") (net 4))
 (segment (start 190.9 113.025) (end 172.875 95) (width 1) (layer "F.Cu") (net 4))
 (segment (start 148.9 91.8) (end 148.9 95) (width 1) (layer "F.Cu") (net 4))
 (segment (start 172.875 95) (end 166.5 95) (width 1) (layer "F.Cu") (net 4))
 (segment (start 190.9 138.4) (end 190.9 113.025) (width 1) (layer "F.Cu") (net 4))
 (segment (start 190.9 138.6) (end 191 138.5) (width 0.2) (layer "F.Cu") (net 4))
 (segment (start 166.5 95) (end 167 95) (width 1) (layer "F.Cu") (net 4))
 (segment (start 190.9 142.3) (end 190.9 138.6) (width 1) (layer "F.Cu") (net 4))
 (via blind (at 166.5 95) (size 1) (drill 0.4) (layers "F.Cu" "B.Cu") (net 4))
 (via blind (at 148.9 95) (size 1) (drill 0.4) (layers "F.Cu" "B.Cu") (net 4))
 (segment (start 166.5 95) (end 148.9 95) (width 1) (layer "B.Cu") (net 4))
 (segment (start 148.9 95) (end 150.75 95) (width 1) (layer "B.Cu") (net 4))
 (segment (start 196 99.25) (end 190.9 94.15) (width 1) (layer "F.Cu") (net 3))
 (segment (start 196 131) (end 196 99.25) (width 1) (layer "F.Cu") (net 3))
 (segment (start 190.9 90.573448) (end 190.94676 90.565203) (width 1) (layer "F.Cu") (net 3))
 (segment (start 190.9 94.15) (end 190.9 90.573448) (width 1) (layer "F.Cu") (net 3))
 (segment (start 194.4 132.6) (end 196 131) (width 1) (layer "F.Cu") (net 3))
 (segment (start 194.4 142.3) (end 194.4 132.6) (width 1) (layer "F.Cu") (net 3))
 (segment (start 201.4 142.3) (end 201.4 97.365835) (width 1) (layer "F.Cu") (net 1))
 (segment (start 201.4 97.365835) (end 197.9 93.865835) (width 1) (layer "F.Cu") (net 1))
 (segment (start 197.9 90.555815) (end 197.946763 90.565202) (width 1) (layer "F.Cu") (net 1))
 (segment (start 197.9 93.865835) (end 197.9 90.555815) (width 1) (layer "F.Cu") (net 1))
 (segment (start 145.4 142.3) (end 145.4 142) (width 0.2) (layer "F.Cu") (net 15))
 (segment (start 145.4 141.35) (end 145.4 142) (width 1) (layer "F.Cu") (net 15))
 (segment (start 141.9 119.8) (end 146.25 119.8) (width 1) (layer "F.Cu") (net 15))
 (segment (start 148.198122 138.551878) (end 145.4 141.35) (width 1) (layer "F.Cu") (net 15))
 (segment (start 148.199446 138.551878) (end 148.198122 138.551878) (width 1) (layer "F.Cu") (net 15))
 (via blind (at 148.199446 138.551878) (size 1) (drill 0.4) (layers "F.Cu" "B.Cu") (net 15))
 (via blind (at 146.25 119.8) (size 1) (drill 0.4) (layers "F.Cu" "B.Cu") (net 15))
 (segment (start 148.199446 138.551878) (end 148.199446 138.550554) (width 1) (layer "B.Cu") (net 15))
 (segment (start 148.199446 138.550554) (end 149 137.75) (width 1) (layer "B.Cu") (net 15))
 (segment (start 149 137.75) (end 149 121.25) (width 1) (layer "B.Cu") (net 15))
 (segment (start 149 121.25) (end 147.55 119.8) (width 1) (layer "B.Cu") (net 15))
 (segment (start 147.55 119.8) (end 146.25 119.8) (width 1) (layer "B.Cu") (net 15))
 (segment (start 169.669805 102.5) (end 160.828623 102.5) (width 1) (layer "F.Cu") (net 6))
 (segment (start 183.9 116.730195) (end 169.669805 102.5) (width 1) (layer "F.Cu") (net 6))
 (segment (start 155.9 90.611965) (end 155.946762 90.565203) (width 1) (layer "F.Cu") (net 6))
 (segment (start 183.9 142.3) (end 183.9 116.730195) (width 1) (layer "F.Cu") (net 6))
 (segment (start 160.828623 102.5) (end 155.9 97.571377) (width 1) (layer "F.Cu") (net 6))
 (segment (start 155.9 97.571377) (end 155.9 90.611965) (width 1) (layer "F.Cu") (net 6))
 (segment (start 197.9 132.85) (end 198.733453 132.016547) (width 1) (layer "F.Cu") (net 2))
 (segment (start 198.733453 98.298152) (end 194.4 93.964699) (width 1) (layer "F.Cu") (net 2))
 (segment (start 198.733453 132.016547) (end 198.733453 98.298152) (width 1) (layer "F.Cu") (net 2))
 (segment (start 197.9 142.3) (end 197.9 132.85) (width 1) (layer "F.Cu") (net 2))
 (segment (start 194.4 93.964699) (end 194.4 90.611965) (width 1) (layer "F.Cu") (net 2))
 (segment (start 194.4 90.611965) (end 194.446762 90.565203) (width 1) (layer "F.Cu") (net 2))
 (segment (start 164 112) (end 156.814252 112) (width 1) (layer "F.Cu") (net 9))
 (segment (start 173.4 121.4) (end 164 112) (width 1) (layer "F.Cu") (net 9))
 (segment (start 156.814252 112) (end 150.56749 105.753238) (width 1) (layer "F.Cu") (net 9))
 (segment (start 173.4 142.3) (end 173.4 121.4) (width 1) (layer "F.Cu") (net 9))
 (segment (start 150.56749 105.753238) (end 142.165203 105.753238) (width 1) (layer "F.Cu") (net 9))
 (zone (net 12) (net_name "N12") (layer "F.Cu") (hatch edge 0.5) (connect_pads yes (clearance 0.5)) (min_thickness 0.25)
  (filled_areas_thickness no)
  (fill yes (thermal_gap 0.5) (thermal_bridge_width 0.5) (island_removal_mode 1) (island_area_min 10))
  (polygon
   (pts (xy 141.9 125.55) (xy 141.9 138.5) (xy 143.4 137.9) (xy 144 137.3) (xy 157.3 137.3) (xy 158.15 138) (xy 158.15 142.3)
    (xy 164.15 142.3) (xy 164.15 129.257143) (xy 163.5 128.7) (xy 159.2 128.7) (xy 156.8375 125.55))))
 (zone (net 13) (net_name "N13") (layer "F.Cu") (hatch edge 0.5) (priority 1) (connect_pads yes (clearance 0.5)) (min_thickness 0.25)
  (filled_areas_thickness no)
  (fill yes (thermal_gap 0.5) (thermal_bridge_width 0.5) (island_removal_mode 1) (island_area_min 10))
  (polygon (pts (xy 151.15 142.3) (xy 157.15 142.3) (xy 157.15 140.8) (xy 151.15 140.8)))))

